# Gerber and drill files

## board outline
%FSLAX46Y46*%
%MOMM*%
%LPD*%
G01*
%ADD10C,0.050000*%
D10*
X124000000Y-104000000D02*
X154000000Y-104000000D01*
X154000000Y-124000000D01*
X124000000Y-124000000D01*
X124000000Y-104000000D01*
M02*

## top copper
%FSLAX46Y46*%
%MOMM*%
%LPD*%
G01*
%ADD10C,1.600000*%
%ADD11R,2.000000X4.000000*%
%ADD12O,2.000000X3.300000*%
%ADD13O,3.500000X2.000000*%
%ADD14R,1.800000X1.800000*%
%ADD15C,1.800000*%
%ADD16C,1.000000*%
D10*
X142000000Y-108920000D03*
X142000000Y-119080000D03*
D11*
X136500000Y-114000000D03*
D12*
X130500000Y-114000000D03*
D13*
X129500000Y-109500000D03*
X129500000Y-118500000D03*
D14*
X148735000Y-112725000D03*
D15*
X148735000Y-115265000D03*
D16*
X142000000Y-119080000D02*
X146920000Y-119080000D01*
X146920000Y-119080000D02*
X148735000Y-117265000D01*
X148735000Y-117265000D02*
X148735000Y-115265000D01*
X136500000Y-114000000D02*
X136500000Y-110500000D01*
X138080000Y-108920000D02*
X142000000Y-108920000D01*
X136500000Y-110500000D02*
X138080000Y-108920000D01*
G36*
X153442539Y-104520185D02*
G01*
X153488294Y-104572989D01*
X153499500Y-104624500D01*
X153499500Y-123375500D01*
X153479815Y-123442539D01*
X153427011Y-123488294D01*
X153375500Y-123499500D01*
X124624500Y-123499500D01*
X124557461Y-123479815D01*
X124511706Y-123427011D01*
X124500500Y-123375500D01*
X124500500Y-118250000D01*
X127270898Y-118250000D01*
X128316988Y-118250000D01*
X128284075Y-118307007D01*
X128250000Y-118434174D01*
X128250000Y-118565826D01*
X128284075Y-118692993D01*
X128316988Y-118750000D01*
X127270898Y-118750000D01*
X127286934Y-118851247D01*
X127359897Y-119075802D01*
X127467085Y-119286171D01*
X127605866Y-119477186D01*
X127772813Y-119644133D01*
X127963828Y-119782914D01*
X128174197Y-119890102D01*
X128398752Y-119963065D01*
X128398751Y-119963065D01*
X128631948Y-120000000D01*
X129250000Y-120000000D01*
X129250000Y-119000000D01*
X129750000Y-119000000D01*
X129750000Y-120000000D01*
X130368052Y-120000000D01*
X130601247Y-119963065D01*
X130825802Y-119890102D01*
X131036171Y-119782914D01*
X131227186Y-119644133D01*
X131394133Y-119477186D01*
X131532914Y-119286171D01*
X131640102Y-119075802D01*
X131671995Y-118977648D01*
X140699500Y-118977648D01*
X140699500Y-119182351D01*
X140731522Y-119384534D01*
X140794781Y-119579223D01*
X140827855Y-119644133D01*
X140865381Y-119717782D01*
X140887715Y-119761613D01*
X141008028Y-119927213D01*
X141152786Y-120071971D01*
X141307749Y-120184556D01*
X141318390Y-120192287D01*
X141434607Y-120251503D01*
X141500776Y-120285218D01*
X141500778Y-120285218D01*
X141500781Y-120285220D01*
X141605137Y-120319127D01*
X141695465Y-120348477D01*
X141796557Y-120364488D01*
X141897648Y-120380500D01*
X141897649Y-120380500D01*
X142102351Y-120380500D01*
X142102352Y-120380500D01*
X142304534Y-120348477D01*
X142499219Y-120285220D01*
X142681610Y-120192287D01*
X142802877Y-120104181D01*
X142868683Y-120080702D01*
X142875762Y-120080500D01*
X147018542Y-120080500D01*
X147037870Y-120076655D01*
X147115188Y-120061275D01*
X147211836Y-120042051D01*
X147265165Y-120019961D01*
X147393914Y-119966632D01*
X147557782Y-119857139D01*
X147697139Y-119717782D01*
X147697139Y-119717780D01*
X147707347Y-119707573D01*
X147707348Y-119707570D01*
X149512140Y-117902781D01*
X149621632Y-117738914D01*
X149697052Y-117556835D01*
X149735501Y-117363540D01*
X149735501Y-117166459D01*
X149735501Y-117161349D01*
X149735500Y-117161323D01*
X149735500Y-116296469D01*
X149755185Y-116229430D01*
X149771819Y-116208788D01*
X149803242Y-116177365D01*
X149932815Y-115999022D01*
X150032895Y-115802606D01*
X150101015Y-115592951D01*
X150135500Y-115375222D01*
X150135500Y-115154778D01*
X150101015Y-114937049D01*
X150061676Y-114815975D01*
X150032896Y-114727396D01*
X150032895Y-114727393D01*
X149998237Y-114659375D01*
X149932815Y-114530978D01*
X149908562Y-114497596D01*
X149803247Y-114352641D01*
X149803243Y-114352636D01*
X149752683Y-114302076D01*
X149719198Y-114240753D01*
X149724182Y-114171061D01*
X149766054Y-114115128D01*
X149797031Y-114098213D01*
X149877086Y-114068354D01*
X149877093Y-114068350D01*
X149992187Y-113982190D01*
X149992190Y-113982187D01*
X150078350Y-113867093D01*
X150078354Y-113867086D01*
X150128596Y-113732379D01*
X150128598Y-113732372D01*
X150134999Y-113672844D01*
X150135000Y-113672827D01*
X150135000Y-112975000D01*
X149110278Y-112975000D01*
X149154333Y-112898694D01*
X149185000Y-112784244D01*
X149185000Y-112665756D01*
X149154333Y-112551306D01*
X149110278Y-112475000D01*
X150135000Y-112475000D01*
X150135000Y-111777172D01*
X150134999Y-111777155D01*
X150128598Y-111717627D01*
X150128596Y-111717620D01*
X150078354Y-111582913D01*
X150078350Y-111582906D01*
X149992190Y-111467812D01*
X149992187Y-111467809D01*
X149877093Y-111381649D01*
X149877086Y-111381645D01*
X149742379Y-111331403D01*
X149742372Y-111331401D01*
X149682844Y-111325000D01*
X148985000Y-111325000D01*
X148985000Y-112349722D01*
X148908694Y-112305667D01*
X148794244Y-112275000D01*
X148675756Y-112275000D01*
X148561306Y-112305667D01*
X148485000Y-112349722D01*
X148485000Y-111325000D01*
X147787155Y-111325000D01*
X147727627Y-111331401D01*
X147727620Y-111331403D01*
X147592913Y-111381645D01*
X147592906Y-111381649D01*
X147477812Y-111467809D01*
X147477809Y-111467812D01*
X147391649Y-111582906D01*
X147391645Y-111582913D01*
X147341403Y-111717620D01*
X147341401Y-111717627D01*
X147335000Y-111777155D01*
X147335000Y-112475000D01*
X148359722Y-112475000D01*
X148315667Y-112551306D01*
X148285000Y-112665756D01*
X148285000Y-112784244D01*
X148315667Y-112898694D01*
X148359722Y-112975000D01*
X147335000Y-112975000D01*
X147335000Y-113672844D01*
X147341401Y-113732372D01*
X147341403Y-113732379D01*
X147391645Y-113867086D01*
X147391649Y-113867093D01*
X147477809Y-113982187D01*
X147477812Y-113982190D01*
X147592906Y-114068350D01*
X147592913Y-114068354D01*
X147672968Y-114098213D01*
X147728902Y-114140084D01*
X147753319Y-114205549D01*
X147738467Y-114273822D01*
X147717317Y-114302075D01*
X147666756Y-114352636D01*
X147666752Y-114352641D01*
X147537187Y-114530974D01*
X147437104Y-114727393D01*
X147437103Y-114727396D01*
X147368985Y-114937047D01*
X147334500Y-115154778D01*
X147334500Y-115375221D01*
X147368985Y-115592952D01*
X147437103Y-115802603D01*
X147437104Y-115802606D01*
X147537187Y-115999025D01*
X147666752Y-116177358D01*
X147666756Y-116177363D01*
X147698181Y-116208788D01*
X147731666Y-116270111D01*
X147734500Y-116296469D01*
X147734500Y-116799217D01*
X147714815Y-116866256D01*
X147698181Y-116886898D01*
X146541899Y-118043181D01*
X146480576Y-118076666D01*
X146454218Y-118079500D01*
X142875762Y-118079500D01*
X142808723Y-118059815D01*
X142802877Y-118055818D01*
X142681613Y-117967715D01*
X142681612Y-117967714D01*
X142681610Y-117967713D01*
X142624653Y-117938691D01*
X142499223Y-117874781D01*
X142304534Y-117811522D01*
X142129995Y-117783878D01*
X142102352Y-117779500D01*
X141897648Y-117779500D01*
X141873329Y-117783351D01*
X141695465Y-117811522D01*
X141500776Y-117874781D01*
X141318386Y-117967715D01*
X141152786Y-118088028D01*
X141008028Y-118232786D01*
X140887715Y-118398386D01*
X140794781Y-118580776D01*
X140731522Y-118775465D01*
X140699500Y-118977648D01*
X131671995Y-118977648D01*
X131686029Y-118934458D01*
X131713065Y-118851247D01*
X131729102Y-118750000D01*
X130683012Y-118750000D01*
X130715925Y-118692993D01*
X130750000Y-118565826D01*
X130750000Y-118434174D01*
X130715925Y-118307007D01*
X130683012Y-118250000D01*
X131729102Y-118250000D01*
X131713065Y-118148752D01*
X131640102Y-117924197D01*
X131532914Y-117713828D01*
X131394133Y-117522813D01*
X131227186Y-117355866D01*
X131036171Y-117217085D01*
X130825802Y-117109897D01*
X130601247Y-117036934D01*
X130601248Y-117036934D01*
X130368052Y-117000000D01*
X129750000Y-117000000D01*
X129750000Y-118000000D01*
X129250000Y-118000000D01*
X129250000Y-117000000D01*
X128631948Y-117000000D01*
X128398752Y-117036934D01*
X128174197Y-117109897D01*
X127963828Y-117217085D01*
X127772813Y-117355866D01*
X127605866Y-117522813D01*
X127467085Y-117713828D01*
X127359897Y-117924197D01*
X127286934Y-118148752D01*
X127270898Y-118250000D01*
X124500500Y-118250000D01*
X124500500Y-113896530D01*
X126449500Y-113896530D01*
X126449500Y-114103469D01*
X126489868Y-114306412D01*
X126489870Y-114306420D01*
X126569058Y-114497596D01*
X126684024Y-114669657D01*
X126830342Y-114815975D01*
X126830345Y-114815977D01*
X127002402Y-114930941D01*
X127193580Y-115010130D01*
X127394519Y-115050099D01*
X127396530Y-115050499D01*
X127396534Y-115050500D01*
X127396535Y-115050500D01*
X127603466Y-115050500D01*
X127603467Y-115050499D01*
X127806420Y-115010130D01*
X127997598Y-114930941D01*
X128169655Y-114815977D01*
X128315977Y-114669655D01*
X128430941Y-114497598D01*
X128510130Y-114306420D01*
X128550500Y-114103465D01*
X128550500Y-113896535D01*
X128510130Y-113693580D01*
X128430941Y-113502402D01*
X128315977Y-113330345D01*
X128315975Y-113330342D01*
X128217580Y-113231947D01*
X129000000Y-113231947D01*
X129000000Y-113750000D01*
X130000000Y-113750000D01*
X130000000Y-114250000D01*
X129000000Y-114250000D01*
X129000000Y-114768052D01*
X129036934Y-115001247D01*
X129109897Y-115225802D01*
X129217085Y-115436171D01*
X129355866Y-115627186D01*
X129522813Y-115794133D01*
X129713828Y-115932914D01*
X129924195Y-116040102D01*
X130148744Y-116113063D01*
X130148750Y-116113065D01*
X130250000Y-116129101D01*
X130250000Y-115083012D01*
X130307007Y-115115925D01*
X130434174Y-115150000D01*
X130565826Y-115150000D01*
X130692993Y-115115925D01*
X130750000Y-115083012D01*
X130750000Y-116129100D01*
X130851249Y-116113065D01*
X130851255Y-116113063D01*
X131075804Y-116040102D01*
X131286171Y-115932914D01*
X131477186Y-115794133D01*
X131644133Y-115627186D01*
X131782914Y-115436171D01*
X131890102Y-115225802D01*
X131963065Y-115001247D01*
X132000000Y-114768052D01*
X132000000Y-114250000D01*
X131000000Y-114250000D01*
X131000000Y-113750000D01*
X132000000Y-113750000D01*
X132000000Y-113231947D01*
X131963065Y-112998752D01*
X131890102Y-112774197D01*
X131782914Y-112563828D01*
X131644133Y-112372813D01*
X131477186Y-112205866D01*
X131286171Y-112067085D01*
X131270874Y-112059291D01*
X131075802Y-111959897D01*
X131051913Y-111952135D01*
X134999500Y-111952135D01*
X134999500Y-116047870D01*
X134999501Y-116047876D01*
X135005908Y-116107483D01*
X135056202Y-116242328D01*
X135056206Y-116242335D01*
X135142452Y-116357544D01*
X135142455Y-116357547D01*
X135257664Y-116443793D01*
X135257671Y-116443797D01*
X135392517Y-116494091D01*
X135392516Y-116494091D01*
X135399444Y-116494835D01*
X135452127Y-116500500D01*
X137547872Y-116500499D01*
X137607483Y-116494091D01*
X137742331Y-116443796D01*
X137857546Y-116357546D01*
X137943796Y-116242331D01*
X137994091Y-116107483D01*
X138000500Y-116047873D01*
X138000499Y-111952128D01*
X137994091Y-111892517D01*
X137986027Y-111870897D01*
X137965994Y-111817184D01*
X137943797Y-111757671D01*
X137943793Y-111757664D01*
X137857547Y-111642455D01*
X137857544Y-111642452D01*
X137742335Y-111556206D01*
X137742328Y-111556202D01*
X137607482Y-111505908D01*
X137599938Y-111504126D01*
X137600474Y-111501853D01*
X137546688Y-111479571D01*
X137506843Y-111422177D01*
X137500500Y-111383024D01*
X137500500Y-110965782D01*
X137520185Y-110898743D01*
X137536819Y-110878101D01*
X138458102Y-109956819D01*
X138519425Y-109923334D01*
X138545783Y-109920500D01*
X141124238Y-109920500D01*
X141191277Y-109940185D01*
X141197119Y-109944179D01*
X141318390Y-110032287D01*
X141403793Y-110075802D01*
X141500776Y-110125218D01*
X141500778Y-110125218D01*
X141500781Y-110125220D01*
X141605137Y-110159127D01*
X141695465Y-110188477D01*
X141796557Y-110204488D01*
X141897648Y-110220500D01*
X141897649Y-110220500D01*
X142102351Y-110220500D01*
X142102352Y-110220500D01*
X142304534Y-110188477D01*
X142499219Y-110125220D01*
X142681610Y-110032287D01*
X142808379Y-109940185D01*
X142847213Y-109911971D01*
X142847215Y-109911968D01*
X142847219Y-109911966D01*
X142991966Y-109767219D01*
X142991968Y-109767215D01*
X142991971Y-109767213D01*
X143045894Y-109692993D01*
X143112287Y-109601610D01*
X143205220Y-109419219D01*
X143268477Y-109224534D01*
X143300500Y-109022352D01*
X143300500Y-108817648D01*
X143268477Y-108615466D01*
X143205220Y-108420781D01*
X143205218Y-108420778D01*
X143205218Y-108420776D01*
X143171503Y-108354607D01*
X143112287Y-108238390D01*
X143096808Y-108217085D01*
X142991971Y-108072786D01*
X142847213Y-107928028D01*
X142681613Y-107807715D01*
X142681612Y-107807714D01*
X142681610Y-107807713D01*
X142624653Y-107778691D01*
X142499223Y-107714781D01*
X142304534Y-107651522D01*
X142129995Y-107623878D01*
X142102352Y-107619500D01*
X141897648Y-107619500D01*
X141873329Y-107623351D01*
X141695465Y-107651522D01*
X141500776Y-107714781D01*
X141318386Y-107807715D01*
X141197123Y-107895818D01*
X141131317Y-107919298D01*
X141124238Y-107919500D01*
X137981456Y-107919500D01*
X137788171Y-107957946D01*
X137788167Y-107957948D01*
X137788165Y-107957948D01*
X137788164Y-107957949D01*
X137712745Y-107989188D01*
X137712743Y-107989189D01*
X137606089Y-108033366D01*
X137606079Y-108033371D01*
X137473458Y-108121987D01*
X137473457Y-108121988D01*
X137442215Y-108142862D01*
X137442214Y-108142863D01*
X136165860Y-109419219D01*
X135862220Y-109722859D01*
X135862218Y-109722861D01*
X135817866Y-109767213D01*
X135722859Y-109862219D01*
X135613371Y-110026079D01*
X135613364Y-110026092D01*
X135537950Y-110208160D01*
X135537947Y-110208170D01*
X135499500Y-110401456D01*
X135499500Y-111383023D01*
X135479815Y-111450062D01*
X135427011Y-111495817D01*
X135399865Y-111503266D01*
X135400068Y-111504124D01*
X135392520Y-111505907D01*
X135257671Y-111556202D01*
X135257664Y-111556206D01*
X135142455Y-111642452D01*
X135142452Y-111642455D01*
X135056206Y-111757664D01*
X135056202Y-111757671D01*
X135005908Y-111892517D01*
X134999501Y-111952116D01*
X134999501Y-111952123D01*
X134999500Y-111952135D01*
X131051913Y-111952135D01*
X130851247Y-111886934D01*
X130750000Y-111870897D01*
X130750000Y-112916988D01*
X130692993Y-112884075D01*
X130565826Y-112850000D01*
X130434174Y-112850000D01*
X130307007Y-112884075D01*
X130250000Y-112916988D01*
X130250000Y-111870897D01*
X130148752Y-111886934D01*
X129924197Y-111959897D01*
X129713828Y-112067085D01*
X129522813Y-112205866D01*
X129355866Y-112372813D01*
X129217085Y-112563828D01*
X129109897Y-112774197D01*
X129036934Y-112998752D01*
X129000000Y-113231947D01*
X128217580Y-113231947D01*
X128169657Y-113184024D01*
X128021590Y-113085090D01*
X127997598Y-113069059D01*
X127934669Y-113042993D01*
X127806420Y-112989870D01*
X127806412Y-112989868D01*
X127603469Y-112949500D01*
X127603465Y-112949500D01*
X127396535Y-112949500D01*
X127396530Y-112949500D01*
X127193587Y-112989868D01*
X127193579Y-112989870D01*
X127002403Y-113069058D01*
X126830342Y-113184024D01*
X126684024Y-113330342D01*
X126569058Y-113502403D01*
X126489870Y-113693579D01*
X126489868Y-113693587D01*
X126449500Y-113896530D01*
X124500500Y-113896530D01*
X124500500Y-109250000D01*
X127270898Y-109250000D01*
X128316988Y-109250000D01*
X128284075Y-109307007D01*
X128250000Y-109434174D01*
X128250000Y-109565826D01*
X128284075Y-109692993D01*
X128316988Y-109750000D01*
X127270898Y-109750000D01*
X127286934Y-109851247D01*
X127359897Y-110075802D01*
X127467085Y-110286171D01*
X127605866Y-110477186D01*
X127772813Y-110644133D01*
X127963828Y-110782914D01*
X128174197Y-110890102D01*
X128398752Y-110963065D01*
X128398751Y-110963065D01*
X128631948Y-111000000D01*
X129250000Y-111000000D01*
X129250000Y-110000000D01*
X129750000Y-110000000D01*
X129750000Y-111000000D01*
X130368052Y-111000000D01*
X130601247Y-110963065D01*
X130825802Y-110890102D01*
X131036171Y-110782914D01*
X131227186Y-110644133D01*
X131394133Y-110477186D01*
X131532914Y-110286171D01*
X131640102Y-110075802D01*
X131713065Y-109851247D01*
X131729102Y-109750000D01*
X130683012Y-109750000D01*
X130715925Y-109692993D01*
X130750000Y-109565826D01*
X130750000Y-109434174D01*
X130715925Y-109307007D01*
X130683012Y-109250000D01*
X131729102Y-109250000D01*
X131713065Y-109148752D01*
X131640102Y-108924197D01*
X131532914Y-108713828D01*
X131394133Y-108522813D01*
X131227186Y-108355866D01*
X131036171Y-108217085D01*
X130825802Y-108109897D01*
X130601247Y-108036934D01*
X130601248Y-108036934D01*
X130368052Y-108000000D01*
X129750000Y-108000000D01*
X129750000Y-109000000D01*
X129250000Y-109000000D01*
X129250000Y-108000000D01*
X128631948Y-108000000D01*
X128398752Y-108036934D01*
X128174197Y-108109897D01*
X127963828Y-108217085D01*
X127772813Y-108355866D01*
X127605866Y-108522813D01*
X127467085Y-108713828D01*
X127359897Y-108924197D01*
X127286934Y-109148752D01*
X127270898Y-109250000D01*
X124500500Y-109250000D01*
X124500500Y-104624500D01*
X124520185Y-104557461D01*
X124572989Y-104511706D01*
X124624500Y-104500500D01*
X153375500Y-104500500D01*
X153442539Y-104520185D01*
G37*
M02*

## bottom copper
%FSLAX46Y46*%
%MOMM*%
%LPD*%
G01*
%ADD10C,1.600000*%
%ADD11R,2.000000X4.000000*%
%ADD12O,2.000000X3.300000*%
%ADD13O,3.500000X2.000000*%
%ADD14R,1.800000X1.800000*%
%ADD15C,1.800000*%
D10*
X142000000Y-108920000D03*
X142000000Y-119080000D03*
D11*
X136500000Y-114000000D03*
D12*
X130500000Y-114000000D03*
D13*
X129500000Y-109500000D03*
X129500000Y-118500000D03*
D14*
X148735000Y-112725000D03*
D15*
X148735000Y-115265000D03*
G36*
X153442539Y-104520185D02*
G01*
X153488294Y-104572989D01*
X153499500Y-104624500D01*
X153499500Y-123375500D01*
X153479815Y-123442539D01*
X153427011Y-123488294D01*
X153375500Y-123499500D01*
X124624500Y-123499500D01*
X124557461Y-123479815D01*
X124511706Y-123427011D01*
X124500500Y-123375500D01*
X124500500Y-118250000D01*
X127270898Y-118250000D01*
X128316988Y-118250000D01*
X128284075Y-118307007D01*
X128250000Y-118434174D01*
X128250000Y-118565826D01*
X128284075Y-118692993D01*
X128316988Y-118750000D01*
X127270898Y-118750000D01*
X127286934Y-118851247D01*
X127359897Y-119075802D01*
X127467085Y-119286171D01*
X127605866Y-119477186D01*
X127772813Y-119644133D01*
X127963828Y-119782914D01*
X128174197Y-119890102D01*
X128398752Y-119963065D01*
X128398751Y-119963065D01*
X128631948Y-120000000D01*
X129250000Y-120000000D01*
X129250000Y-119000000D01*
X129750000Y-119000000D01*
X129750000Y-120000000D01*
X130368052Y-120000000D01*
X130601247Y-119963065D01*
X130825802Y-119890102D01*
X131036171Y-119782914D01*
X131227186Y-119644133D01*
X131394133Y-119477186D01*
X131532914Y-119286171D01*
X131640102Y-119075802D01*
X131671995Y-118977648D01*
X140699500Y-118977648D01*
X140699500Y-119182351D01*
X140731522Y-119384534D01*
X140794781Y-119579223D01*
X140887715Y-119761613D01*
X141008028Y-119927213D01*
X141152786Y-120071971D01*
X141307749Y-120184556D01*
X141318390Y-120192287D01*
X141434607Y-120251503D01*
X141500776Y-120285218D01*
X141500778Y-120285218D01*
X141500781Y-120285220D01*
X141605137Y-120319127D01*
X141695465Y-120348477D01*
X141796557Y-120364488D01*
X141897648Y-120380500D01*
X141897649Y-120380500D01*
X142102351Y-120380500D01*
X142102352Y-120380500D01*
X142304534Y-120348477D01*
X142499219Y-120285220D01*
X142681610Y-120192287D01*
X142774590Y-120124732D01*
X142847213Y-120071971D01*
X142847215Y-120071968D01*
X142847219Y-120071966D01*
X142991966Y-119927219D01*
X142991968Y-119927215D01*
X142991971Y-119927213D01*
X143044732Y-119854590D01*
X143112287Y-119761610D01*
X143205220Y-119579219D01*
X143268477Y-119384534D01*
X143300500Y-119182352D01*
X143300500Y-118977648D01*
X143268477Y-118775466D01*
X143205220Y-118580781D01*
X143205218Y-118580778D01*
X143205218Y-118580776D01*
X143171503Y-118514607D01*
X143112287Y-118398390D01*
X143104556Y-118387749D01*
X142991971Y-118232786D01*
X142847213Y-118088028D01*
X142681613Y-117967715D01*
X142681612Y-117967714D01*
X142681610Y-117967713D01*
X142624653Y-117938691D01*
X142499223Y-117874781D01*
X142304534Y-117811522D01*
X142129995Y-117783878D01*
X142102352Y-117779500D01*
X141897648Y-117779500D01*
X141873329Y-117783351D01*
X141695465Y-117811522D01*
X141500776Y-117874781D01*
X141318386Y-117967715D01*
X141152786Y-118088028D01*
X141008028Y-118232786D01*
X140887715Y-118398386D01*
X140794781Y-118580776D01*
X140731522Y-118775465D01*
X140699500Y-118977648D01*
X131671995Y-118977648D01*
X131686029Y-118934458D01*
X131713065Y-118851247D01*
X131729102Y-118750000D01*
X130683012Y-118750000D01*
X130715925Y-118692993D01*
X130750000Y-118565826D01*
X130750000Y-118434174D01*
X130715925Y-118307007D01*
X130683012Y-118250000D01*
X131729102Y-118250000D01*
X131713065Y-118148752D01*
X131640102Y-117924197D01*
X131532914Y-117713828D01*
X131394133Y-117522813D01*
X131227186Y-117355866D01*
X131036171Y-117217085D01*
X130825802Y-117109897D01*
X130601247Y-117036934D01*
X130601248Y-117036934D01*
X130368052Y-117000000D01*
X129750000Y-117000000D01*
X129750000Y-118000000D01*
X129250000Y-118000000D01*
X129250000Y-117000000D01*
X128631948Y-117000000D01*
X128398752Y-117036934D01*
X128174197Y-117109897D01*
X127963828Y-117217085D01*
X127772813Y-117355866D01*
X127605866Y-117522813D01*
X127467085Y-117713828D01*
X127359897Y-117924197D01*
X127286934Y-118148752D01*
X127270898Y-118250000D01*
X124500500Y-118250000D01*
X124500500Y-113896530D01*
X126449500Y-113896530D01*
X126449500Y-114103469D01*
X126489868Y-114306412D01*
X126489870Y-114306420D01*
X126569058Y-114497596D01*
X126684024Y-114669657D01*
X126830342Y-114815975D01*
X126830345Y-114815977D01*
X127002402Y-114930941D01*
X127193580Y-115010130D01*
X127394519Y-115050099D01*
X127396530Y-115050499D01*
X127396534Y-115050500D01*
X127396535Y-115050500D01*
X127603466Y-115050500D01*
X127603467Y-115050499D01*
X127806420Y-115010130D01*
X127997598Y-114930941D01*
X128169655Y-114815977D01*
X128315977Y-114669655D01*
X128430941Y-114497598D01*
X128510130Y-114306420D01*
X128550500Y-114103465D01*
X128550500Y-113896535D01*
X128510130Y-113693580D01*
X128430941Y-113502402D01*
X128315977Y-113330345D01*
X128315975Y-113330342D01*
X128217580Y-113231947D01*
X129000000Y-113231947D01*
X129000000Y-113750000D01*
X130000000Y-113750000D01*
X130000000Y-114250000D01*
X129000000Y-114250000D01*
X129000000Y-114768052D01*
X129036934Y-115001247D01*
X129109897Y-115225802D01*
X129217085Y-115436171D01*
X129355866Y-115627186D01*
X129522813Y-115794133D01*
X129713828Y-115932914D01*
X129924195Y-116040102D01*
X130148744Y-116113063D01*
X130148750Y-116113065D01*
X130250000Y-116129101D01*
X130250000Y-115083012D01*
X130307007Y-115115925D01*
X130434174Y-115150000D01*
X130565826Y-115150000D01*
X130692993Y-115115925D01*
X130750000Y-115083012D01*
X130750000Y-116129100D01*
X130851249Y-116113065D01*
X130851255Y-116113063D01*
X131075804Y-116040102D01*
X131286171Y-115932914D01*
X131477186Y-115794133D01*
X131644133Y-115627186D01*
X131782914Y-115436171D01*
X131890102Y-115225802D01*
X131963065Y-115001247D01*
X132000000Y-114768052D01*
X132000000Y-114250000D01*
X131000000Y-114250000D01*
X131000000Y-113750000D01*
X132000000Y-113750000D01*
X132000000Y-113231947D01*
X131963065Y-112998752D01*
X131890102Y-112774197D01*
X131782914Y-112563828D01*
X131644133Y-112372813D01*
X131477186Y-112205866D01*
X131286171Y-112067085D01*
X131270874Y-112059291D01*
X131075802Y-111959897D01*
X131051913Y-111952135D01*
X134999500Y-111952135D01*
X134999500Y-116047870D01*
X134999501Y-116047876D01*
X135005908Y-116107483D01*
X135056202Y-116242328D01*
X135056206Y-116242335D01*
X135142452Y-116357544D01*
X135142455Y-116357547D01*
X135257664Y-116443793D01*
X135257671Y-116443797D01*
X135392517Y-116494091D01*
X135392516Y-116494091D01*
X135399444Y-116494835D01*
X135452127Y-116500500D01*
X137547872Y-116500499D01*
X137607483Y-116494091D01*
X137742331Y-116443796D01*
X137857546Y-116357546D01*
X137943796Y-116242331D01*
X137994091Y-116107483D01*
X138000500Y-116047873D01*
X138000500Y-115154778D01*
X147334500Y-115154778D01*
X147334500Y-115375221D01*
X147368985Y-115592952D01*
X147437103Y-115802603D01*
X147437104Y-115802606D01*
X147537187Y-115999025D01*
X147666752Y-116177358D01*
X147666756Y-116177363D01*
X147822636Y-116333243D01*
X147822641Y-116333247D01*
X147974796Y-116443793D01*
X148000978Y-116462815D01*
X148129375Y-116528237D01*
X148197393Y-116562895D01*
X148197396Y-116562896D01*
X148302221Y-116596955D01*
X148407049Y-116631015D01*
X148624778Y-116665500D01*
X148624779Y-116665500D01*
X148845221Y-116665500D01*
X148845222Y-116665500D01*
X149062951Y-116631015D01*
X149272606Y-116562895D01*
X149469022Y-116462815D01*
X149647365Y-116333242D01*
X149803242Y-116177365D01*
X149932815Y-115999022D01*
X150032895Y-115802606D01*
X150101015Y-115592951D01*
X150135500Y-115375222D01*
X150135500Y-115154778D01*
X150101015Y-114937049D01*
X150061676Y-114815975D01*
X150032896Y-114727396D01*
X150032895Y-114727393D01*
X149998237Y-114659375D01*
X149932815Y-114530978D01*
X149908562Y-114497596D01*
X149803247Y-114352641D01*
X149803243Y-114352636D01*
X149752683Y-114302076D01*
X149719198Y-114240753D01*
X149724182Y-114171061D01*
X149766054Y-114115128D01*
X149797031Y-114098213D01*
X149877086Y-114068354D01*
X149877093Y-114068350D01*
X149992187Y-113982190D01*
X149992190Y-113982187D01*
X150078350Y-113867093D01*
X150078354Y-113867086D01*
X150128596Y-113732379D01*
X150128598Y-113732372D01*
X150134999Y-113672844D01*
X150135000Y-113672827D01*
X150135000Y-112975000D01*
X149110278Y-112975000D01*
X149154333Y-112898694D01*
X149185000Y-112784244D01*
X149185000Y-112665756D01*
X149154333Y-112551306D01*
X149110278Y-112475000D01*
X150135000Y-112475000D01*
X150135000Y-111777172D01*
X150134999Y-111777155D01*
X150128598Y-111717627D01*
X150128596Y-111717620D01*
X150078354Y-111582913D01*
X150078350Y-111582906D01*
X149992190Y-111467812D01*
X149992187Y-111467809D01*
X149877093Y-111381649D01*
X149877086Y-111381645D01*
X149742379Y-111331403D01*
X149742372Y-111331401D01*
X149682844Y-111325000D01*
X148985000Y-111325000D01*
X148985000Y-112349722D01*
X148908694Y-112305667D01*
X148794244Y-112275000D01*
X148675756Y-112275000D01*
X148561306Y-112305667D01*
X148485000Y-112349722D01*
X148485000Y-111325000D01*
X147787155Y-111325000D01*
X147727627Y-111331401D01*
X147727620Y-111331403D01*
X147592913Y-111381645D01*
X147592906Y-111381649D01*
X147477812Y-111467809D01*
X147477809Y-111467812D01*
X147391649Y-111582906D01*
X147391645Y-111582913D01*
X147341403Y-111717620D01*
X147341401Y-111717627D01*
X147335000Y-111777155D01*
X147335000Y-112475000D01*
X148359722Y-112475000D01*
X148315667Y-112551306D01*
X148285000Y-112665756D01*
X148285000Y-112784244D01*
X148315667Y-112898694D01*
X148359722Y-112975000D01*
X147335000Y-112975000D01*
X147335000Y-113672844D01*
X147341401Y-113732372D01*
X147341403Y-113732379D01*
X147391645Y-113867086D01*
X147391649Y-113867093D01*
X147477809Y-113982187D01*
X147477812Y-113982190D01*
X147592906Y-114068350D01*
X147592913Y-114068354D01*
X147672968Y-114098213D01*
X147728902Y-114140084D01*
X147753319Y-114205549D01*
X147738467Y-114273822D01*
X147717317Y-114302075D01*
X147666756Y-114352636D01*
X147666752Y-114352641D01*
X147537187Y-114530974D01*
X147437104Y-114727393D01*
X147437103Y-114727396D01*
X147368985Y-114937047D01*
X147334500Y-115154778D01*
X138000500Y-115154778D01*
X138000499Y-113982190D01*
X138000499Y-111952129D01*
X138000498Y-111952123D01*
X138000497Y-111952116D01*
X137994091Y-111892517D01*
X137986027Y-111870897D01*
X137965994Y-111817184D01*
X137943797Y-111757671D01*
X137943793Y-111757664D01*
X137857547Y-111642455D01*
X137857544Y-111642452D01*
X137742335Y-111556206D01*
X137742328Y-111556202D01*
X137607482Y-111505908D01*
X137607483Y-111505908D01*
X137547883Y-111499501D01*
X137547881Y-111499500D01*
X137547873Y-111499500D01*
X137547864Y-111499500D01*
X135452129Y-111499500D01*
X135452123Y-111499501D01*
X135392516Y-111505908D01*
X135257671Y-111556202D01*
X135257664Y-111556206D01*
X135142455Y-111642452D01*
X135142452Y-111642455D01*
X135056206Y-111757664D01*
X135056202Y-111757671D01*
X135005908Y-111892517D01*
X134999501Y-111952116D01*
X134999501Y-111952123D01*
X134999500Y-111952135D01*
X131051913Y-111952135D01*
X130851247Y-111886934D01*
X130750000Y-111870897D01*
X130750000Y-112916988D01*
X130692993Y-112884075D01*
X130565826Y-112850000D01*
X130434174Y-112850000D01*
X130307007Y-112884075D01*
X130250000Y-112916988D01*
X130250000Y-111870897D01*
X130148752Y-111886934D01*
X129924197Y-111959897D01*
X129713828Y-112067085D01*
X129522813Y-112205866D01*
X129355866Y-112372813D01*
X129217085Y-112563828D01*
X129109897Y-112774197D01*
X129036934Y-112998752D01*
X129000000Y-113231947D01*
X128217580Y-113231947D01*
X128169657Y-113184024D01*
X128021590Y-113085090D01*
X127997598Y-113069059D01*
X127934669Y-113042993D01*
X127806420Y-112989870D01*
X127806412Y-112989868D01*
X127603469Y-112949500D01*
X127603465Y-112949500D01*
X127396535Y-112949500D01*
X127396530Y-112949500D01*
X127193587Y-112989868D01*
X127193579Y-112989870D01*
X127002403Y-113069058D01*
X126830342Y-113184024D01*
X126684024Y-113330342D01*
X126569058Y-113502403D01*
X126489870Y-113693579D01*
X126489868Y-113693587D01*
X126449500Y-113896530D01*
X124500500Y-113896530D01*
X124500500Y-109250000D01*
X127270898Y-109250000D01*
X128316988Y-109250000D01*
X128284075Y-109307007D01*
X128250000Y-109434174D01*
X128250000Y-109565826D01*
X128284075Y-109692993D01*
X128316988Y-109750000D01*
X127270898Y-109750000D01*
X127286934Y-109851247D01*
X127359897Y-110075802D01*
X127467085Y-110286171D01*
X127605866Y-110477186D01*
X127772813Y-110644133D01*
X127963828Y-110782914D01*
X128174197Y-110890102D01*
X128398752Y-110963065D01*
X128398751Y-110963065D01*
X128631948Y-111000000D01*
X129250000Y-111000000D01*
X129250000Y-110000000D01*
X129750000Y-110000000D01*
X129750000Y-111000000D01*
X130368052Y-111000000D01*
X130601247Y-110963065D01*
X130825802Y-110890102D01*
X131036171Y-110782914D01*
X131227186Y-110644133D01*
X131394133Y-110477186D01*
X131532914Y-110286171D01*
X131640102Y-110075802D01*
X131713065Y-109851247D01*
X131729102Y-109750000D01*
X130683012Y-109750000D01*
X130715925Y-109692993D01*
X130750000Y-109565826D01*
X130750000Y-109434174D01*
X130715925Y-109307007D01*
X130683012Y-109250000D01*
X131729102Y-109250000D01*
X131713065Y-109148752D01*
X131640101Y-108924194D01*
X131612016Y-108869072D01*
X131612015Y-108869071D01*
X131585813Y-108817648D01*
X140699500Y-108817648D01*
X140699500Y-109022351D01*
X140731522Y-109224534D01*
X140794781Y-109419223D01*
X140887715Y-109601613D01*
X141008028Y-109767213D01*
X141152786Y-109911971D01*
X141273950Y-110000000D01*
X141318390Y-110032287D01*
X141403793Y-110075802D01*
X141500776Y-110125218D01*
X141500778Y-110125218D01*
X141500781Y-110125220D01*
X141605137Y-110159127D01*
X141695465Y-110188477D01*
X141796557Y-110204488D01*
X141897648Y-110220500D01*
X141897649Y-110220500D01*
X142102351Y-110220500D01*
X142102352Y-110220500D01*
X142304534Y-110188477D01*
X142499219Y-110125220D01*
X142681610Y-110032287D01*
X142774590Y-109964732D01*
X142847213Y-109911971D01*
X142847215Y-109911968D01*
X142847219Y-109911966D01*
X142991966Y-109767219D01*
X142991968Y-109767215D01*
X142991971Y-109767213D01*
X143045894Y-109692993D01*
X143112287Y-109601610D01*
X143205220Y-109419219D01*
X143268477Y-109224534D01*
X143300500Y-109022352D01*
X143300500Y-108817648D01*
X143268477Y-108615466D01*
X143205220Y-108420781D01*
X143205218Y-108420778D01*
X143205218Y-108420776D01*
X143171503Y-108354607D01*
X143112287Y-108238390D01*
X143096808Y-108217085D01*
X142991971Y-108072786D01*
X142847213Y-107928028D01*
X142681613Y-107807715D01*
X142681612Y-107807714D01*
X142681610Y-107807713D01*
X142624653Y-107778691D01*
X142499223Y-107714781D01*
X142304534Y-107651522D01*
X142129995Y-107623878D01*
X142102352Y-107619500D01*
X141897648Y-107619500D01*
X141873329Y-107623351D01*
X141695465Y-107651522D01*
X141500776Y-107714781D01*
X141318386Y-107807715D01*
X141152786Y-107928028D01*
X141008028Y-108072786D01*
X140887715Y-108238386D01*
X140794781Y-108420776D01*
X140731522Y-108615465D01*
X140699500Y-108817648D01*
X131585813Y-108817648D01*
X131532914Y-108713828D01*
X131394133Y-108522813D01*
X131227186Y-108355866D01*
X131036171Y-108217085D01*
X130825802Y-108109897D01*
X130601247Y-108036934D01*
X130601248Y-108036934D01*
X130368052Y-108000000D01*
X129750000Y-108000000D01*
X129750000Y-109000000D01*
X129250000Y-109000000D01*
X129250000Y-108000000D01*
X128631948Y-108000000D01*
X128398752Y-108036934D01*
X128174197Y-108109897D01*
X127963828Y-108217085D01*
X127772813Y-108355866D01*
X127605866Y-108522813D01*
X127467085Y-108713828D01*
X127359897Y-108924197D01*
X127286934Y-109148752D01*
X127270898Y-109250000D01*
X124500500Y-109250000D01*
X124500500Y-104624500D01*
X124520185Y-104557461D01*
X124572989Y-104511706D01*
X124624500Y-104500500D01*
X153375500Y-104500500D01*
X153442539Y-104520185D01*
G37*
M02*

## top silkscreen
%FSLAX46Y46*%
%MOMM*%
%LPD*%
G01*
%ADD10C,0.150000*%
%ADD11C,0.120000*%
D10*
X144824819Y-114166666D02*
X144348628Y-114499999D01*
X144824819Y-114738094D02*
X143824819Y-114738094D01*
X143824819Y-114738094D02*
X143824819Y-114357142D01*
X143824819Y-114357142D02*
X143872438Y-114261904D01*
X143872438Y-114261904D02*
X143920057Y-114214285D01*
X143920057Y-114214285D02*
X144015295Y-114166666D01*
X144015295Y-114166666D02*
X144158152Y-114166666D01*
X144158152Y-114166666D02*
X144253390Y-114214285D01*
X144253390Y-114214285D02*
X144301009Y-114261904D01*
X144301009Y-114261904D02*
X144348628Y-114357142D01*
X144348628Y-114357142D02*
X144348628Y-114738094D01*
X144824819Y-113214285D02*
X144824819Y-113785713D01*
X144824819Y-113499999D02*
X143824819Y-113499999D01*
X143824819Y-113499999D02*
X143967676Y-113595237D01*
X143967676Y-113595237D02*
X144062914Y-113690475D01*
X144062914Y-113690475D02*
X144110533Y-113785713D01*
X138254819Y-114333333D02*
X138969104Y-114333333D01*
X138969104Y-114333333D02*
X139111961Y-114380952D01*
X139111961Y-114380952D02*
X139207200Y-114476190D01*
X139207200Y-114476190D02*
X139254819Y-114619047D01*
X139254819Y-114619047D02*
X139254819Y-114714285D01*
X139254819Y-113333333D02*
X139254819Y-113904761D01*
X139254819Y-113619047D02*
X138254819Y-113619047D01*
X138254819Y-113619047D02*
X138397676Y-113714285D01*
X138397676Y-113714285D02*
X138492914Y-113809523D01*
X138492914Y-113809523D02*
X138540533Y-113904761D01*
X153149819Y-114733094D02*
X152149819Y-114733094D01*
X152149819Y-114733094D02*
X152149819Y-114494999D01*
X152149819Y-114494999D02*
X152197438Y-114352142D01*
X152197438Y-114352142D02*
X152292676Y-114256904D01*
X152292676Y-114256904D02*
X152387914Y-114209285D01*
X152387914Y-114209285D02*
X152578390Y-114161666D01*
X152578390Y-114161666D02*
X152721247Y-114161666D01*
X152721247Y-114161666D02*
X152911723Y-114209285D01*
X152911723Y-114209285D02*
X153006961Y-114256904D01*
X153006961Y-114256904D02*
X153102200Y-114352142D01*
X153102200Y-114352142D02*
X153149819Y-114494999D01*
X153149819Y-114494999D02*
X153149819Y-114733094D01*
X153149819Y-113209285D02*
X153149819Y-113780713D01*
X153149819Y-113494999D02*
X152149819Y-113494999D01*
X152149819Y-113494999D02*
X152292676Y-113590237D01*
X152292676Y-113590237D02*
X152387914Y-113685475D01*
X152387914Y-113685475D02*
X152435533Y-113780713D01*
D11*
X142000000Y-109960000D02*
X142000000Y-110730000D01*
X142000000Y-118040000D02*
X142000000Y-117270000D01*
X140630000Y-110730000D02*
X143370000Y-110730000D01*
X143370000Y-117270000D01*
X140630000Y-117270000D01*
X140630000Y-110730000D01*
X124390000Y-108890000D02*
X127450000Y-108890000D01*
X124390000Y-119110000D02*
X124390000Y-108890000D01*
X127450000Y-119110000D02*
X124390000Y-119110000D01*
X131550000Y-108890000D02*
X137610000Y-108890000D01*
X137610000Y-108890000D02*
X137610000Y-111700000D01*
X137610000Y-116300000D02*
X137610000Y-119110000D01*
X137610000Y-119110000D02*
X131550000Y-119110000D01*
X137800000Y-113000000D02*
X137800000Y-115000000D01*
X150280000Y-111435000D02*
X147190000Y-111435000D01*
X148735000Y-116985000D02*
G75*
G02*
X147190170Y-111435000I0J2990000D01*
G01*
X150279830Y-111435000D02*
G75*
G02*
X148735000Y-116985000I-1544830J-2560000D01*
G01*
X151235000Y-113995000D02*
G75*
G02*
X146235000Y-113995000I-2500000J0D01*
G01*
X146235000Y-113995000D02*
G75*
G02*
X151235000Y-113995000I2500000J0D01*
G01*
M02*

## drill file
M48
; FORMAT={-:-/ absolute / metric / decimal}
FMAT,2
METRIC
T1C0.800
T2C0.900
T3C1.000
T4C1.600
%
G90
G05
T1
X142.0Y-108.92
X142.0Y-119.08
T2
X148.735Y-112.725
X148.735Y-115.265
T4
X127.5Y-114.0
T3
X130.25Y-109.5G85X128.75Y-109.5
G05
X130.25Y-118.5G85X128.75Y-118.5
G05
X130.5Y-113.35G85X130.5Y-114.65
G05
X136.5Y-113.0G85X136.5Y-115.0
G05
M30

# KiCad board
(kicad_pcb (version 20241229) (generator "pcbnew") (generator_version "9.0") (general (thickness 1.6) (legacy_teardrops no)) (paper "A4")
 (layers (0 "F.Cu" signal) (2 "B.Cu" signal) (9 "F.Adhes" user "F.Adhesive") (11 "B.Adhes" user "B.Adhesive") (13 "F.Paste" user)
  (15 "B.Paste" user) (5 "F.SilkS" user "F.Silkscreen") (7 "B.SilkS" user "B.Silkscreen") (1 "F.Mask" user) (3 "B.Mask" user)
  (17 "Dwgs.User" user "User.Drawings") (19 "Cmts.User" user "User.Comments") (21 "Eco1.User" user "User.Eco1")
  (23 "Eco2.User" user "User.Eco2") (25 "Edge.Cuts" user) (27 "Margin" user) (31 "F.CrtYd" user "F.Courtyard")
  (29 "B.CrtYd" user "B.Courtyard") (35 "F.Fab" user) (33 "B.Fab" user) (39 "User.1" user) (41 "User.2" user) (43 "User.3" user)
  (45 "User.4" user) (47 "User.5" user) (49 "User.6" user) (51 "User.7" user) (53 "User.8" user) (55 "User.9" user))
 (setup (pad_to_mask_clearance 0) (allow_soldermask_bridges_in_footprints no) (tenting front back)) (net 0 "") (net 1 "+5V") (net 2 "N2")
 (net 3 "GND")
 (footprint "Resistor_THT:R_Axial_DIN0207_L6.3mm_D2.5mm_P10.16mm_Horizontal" (layer "F.Cu") (at 142 108.92 -90)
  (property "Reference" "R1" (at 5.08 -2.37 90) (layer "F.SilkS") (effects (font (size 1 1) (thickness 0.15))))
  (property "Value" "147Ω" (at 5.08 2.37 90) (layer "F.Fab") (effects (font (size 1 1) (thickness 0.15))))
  (fp_line (start 1.04 0) (end 1.81 0) (stroke (width 0.12) (type solid)) (layer "F.SilkS"))
  (fp_line (start 9.12 0) (end 8.35 0) (stroke (width 0.12) (type solid)) (layer "F.SilkS"))
  (fp_rect (start 1.81 -1.37) (end 8.35 1.37) (stroke (width 0.12) (type solid)) (fill no) (layer "F.SilkS"))
  (pad "1" thru_hole circle (at 0 0 270) (size 1.6 1.6) (drill 0.8) (layers "*.Cu" "*.Mask") (remove_unused_layers no) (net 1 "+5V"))
  (pad "2" thru_hole circle (at 10.16 0 270) (size 1.6 1.6) (drill 0.8) (layers "*.Cu" "*.Mask") (remove_unused_layers no) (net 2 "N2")))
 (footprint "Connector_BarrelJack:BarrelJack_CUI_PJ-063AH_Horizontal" (layer "F.Cu") (at 136.5 114 -90)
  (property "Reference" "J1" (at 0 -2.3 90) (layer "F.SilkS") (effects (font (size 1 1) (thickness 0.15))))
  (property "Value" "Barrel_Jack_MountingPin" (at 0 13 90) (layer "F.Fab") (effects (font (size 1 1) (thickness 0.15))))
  (fp_line (start -5.11 12.11) (end -5.11 9.05) (stroke (width 0.12) (type solid)) (layer "F.SilkS"))
  (fp_line (start 5.11 12.11) (end -5.11 12.11) (stroke (width 0.12) (type solid)) (layer "F.SilkS"))
  (fp_line (start 5.11 9.05) (end 5.11 12.11) (stroke (width 0.12) (type solid)) (layer "F.SilkS"))
  (fp_line (start -5.11 4.95) (end -5.11 -1.11) (stroke (width 0.12) (type solid)) (layer "F.SilkS"))
  (fp_line (start -5.11 -1.11) (end -2.3 -1.11) (stroke (width 0.12) (type solid)) (layer "F.SilkS"))
  (fp_line (start 2.3 -1.11) (end 5.11 -1.11) (stroke (width 0.12) (type solid)) (layer "F.SilkS"))
  (fp_line (start 5.11 -1.11) (end 5.11 4.95) (stroke (width 0.12) (type solid)) (layer "F.SilkS"))
  (fp_line (start -1 -1.3) (end 1 -1.3) (stroke (width 0.12) (type solid)) (layer "F.SilkS"))
  (pad "" np_thru_hole circle (at 0 9 270) (size 1.6 1.6) (drill 1.6) (layers "*.Cu" "*.Mask"))
  (pad "1" thru_hole rect (at 0 0 270) (size 4 2) (drill oval 3 1) (layers "*.Cu" "*.Mask") (remove_unused_layers no) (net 1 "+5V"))
  (pad "2" thru_hole oval (at 0 6 270) (size 3.3 2) (drill oval 2.3 1) (layers "*.Cu" "*.Mask") (remove_unused_layers no) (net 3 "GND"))
  (pad "MP" thru_hole oval (at -4.5 7 270) (size 2 3.5) (drill oval 1 2.5) (layers "*.Cu" "*.Mask") (remove_unused_layers no) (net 3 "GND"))
  (pad "MP" thru_hole oval (at 4.5 7 270) (size 2 3.5) (drill oval 1 2.5) (layers "*.Cu" "*.Mask") (remove_unused_layers no) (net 3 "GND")))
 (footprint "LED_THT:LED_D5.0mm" (layer "F.Cu") (at 148.735 112.725 -90)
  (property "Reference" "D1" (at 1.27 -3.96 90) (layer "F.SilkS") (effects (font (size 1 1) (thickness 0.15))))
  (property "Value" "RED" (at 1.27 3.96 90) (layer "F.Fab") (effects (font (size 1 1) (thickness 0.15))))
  (fp_line (start -1.29 -1.545) (end -1.29 1.545) (stroke (width 0.12) (type solid)) (layer "F.SilkS"))
  (fp_arc (start 4.26 0) (mid 2.071779 2.880495) (end -1.29 1.54483) (stroke (width 0.12) (type solid)) (layer "F.SilkS"))
  (fp_arc (start -1.29 -1.54483) (mid 2.071779 -2.880495) (end 4.26 0) (stroke (width 0.12) (type solid)) (layer "F.SilkS"))
  (fp_circle (center 1.27 0) (end 3.77 0) (stroke (width 0.12) (type solid)) (fill no) (layer "F.SilkS"))
  (pad "1" thru_hole rect (at 0 0 270) (size 1.8 1.8) (drill 0.9) (layers "*.Cu" "*.Mask") (remove_unused_layers no) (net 3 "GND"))
  (pad "2" thru_hole circle (at 2.54 0 270) (size 1.8 1.8) (drill 0.9) (layers "*.Cu" "*.Mask") (remove_unused_layers no) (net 2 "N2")))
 (gr_rect (start 124 104) (end 154 124) (stroke (width 0.05) (type default)) (fill no) (layer "Edge.Cuts"))
 (segment (start 142 119.08) (end 146.92 119.08) (width 1) (layer "F.Cu") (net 2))
 (segment (start 146.92 119.08) (end 148.735 117.265) (width 1) (layer "F.Cu") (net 2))
 (segment (start 148.735 117.265) (end 148.735 115.265) (width 1) (layer "F.Cu") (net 2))
 (segment (start 136.5 114) (end 136.5 110.5) (width 1) (layer "F.Cu") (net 1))
 (segment (start 138.08 108.92) (end 142 108.92) (width 1) (layer "F.Cu") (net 1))
 (segment (start 136.5 110.5) (end 138.08 108.92) (width 1) (layer "F.Cu") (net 1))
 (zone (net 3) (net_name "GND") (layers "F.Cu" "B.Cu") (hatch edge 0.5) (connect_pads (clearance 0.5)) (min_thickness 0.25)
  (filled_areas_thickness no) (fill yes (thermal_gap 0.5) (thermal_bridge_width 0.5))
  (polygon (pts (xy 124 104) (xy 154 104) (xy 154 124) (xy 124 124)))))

